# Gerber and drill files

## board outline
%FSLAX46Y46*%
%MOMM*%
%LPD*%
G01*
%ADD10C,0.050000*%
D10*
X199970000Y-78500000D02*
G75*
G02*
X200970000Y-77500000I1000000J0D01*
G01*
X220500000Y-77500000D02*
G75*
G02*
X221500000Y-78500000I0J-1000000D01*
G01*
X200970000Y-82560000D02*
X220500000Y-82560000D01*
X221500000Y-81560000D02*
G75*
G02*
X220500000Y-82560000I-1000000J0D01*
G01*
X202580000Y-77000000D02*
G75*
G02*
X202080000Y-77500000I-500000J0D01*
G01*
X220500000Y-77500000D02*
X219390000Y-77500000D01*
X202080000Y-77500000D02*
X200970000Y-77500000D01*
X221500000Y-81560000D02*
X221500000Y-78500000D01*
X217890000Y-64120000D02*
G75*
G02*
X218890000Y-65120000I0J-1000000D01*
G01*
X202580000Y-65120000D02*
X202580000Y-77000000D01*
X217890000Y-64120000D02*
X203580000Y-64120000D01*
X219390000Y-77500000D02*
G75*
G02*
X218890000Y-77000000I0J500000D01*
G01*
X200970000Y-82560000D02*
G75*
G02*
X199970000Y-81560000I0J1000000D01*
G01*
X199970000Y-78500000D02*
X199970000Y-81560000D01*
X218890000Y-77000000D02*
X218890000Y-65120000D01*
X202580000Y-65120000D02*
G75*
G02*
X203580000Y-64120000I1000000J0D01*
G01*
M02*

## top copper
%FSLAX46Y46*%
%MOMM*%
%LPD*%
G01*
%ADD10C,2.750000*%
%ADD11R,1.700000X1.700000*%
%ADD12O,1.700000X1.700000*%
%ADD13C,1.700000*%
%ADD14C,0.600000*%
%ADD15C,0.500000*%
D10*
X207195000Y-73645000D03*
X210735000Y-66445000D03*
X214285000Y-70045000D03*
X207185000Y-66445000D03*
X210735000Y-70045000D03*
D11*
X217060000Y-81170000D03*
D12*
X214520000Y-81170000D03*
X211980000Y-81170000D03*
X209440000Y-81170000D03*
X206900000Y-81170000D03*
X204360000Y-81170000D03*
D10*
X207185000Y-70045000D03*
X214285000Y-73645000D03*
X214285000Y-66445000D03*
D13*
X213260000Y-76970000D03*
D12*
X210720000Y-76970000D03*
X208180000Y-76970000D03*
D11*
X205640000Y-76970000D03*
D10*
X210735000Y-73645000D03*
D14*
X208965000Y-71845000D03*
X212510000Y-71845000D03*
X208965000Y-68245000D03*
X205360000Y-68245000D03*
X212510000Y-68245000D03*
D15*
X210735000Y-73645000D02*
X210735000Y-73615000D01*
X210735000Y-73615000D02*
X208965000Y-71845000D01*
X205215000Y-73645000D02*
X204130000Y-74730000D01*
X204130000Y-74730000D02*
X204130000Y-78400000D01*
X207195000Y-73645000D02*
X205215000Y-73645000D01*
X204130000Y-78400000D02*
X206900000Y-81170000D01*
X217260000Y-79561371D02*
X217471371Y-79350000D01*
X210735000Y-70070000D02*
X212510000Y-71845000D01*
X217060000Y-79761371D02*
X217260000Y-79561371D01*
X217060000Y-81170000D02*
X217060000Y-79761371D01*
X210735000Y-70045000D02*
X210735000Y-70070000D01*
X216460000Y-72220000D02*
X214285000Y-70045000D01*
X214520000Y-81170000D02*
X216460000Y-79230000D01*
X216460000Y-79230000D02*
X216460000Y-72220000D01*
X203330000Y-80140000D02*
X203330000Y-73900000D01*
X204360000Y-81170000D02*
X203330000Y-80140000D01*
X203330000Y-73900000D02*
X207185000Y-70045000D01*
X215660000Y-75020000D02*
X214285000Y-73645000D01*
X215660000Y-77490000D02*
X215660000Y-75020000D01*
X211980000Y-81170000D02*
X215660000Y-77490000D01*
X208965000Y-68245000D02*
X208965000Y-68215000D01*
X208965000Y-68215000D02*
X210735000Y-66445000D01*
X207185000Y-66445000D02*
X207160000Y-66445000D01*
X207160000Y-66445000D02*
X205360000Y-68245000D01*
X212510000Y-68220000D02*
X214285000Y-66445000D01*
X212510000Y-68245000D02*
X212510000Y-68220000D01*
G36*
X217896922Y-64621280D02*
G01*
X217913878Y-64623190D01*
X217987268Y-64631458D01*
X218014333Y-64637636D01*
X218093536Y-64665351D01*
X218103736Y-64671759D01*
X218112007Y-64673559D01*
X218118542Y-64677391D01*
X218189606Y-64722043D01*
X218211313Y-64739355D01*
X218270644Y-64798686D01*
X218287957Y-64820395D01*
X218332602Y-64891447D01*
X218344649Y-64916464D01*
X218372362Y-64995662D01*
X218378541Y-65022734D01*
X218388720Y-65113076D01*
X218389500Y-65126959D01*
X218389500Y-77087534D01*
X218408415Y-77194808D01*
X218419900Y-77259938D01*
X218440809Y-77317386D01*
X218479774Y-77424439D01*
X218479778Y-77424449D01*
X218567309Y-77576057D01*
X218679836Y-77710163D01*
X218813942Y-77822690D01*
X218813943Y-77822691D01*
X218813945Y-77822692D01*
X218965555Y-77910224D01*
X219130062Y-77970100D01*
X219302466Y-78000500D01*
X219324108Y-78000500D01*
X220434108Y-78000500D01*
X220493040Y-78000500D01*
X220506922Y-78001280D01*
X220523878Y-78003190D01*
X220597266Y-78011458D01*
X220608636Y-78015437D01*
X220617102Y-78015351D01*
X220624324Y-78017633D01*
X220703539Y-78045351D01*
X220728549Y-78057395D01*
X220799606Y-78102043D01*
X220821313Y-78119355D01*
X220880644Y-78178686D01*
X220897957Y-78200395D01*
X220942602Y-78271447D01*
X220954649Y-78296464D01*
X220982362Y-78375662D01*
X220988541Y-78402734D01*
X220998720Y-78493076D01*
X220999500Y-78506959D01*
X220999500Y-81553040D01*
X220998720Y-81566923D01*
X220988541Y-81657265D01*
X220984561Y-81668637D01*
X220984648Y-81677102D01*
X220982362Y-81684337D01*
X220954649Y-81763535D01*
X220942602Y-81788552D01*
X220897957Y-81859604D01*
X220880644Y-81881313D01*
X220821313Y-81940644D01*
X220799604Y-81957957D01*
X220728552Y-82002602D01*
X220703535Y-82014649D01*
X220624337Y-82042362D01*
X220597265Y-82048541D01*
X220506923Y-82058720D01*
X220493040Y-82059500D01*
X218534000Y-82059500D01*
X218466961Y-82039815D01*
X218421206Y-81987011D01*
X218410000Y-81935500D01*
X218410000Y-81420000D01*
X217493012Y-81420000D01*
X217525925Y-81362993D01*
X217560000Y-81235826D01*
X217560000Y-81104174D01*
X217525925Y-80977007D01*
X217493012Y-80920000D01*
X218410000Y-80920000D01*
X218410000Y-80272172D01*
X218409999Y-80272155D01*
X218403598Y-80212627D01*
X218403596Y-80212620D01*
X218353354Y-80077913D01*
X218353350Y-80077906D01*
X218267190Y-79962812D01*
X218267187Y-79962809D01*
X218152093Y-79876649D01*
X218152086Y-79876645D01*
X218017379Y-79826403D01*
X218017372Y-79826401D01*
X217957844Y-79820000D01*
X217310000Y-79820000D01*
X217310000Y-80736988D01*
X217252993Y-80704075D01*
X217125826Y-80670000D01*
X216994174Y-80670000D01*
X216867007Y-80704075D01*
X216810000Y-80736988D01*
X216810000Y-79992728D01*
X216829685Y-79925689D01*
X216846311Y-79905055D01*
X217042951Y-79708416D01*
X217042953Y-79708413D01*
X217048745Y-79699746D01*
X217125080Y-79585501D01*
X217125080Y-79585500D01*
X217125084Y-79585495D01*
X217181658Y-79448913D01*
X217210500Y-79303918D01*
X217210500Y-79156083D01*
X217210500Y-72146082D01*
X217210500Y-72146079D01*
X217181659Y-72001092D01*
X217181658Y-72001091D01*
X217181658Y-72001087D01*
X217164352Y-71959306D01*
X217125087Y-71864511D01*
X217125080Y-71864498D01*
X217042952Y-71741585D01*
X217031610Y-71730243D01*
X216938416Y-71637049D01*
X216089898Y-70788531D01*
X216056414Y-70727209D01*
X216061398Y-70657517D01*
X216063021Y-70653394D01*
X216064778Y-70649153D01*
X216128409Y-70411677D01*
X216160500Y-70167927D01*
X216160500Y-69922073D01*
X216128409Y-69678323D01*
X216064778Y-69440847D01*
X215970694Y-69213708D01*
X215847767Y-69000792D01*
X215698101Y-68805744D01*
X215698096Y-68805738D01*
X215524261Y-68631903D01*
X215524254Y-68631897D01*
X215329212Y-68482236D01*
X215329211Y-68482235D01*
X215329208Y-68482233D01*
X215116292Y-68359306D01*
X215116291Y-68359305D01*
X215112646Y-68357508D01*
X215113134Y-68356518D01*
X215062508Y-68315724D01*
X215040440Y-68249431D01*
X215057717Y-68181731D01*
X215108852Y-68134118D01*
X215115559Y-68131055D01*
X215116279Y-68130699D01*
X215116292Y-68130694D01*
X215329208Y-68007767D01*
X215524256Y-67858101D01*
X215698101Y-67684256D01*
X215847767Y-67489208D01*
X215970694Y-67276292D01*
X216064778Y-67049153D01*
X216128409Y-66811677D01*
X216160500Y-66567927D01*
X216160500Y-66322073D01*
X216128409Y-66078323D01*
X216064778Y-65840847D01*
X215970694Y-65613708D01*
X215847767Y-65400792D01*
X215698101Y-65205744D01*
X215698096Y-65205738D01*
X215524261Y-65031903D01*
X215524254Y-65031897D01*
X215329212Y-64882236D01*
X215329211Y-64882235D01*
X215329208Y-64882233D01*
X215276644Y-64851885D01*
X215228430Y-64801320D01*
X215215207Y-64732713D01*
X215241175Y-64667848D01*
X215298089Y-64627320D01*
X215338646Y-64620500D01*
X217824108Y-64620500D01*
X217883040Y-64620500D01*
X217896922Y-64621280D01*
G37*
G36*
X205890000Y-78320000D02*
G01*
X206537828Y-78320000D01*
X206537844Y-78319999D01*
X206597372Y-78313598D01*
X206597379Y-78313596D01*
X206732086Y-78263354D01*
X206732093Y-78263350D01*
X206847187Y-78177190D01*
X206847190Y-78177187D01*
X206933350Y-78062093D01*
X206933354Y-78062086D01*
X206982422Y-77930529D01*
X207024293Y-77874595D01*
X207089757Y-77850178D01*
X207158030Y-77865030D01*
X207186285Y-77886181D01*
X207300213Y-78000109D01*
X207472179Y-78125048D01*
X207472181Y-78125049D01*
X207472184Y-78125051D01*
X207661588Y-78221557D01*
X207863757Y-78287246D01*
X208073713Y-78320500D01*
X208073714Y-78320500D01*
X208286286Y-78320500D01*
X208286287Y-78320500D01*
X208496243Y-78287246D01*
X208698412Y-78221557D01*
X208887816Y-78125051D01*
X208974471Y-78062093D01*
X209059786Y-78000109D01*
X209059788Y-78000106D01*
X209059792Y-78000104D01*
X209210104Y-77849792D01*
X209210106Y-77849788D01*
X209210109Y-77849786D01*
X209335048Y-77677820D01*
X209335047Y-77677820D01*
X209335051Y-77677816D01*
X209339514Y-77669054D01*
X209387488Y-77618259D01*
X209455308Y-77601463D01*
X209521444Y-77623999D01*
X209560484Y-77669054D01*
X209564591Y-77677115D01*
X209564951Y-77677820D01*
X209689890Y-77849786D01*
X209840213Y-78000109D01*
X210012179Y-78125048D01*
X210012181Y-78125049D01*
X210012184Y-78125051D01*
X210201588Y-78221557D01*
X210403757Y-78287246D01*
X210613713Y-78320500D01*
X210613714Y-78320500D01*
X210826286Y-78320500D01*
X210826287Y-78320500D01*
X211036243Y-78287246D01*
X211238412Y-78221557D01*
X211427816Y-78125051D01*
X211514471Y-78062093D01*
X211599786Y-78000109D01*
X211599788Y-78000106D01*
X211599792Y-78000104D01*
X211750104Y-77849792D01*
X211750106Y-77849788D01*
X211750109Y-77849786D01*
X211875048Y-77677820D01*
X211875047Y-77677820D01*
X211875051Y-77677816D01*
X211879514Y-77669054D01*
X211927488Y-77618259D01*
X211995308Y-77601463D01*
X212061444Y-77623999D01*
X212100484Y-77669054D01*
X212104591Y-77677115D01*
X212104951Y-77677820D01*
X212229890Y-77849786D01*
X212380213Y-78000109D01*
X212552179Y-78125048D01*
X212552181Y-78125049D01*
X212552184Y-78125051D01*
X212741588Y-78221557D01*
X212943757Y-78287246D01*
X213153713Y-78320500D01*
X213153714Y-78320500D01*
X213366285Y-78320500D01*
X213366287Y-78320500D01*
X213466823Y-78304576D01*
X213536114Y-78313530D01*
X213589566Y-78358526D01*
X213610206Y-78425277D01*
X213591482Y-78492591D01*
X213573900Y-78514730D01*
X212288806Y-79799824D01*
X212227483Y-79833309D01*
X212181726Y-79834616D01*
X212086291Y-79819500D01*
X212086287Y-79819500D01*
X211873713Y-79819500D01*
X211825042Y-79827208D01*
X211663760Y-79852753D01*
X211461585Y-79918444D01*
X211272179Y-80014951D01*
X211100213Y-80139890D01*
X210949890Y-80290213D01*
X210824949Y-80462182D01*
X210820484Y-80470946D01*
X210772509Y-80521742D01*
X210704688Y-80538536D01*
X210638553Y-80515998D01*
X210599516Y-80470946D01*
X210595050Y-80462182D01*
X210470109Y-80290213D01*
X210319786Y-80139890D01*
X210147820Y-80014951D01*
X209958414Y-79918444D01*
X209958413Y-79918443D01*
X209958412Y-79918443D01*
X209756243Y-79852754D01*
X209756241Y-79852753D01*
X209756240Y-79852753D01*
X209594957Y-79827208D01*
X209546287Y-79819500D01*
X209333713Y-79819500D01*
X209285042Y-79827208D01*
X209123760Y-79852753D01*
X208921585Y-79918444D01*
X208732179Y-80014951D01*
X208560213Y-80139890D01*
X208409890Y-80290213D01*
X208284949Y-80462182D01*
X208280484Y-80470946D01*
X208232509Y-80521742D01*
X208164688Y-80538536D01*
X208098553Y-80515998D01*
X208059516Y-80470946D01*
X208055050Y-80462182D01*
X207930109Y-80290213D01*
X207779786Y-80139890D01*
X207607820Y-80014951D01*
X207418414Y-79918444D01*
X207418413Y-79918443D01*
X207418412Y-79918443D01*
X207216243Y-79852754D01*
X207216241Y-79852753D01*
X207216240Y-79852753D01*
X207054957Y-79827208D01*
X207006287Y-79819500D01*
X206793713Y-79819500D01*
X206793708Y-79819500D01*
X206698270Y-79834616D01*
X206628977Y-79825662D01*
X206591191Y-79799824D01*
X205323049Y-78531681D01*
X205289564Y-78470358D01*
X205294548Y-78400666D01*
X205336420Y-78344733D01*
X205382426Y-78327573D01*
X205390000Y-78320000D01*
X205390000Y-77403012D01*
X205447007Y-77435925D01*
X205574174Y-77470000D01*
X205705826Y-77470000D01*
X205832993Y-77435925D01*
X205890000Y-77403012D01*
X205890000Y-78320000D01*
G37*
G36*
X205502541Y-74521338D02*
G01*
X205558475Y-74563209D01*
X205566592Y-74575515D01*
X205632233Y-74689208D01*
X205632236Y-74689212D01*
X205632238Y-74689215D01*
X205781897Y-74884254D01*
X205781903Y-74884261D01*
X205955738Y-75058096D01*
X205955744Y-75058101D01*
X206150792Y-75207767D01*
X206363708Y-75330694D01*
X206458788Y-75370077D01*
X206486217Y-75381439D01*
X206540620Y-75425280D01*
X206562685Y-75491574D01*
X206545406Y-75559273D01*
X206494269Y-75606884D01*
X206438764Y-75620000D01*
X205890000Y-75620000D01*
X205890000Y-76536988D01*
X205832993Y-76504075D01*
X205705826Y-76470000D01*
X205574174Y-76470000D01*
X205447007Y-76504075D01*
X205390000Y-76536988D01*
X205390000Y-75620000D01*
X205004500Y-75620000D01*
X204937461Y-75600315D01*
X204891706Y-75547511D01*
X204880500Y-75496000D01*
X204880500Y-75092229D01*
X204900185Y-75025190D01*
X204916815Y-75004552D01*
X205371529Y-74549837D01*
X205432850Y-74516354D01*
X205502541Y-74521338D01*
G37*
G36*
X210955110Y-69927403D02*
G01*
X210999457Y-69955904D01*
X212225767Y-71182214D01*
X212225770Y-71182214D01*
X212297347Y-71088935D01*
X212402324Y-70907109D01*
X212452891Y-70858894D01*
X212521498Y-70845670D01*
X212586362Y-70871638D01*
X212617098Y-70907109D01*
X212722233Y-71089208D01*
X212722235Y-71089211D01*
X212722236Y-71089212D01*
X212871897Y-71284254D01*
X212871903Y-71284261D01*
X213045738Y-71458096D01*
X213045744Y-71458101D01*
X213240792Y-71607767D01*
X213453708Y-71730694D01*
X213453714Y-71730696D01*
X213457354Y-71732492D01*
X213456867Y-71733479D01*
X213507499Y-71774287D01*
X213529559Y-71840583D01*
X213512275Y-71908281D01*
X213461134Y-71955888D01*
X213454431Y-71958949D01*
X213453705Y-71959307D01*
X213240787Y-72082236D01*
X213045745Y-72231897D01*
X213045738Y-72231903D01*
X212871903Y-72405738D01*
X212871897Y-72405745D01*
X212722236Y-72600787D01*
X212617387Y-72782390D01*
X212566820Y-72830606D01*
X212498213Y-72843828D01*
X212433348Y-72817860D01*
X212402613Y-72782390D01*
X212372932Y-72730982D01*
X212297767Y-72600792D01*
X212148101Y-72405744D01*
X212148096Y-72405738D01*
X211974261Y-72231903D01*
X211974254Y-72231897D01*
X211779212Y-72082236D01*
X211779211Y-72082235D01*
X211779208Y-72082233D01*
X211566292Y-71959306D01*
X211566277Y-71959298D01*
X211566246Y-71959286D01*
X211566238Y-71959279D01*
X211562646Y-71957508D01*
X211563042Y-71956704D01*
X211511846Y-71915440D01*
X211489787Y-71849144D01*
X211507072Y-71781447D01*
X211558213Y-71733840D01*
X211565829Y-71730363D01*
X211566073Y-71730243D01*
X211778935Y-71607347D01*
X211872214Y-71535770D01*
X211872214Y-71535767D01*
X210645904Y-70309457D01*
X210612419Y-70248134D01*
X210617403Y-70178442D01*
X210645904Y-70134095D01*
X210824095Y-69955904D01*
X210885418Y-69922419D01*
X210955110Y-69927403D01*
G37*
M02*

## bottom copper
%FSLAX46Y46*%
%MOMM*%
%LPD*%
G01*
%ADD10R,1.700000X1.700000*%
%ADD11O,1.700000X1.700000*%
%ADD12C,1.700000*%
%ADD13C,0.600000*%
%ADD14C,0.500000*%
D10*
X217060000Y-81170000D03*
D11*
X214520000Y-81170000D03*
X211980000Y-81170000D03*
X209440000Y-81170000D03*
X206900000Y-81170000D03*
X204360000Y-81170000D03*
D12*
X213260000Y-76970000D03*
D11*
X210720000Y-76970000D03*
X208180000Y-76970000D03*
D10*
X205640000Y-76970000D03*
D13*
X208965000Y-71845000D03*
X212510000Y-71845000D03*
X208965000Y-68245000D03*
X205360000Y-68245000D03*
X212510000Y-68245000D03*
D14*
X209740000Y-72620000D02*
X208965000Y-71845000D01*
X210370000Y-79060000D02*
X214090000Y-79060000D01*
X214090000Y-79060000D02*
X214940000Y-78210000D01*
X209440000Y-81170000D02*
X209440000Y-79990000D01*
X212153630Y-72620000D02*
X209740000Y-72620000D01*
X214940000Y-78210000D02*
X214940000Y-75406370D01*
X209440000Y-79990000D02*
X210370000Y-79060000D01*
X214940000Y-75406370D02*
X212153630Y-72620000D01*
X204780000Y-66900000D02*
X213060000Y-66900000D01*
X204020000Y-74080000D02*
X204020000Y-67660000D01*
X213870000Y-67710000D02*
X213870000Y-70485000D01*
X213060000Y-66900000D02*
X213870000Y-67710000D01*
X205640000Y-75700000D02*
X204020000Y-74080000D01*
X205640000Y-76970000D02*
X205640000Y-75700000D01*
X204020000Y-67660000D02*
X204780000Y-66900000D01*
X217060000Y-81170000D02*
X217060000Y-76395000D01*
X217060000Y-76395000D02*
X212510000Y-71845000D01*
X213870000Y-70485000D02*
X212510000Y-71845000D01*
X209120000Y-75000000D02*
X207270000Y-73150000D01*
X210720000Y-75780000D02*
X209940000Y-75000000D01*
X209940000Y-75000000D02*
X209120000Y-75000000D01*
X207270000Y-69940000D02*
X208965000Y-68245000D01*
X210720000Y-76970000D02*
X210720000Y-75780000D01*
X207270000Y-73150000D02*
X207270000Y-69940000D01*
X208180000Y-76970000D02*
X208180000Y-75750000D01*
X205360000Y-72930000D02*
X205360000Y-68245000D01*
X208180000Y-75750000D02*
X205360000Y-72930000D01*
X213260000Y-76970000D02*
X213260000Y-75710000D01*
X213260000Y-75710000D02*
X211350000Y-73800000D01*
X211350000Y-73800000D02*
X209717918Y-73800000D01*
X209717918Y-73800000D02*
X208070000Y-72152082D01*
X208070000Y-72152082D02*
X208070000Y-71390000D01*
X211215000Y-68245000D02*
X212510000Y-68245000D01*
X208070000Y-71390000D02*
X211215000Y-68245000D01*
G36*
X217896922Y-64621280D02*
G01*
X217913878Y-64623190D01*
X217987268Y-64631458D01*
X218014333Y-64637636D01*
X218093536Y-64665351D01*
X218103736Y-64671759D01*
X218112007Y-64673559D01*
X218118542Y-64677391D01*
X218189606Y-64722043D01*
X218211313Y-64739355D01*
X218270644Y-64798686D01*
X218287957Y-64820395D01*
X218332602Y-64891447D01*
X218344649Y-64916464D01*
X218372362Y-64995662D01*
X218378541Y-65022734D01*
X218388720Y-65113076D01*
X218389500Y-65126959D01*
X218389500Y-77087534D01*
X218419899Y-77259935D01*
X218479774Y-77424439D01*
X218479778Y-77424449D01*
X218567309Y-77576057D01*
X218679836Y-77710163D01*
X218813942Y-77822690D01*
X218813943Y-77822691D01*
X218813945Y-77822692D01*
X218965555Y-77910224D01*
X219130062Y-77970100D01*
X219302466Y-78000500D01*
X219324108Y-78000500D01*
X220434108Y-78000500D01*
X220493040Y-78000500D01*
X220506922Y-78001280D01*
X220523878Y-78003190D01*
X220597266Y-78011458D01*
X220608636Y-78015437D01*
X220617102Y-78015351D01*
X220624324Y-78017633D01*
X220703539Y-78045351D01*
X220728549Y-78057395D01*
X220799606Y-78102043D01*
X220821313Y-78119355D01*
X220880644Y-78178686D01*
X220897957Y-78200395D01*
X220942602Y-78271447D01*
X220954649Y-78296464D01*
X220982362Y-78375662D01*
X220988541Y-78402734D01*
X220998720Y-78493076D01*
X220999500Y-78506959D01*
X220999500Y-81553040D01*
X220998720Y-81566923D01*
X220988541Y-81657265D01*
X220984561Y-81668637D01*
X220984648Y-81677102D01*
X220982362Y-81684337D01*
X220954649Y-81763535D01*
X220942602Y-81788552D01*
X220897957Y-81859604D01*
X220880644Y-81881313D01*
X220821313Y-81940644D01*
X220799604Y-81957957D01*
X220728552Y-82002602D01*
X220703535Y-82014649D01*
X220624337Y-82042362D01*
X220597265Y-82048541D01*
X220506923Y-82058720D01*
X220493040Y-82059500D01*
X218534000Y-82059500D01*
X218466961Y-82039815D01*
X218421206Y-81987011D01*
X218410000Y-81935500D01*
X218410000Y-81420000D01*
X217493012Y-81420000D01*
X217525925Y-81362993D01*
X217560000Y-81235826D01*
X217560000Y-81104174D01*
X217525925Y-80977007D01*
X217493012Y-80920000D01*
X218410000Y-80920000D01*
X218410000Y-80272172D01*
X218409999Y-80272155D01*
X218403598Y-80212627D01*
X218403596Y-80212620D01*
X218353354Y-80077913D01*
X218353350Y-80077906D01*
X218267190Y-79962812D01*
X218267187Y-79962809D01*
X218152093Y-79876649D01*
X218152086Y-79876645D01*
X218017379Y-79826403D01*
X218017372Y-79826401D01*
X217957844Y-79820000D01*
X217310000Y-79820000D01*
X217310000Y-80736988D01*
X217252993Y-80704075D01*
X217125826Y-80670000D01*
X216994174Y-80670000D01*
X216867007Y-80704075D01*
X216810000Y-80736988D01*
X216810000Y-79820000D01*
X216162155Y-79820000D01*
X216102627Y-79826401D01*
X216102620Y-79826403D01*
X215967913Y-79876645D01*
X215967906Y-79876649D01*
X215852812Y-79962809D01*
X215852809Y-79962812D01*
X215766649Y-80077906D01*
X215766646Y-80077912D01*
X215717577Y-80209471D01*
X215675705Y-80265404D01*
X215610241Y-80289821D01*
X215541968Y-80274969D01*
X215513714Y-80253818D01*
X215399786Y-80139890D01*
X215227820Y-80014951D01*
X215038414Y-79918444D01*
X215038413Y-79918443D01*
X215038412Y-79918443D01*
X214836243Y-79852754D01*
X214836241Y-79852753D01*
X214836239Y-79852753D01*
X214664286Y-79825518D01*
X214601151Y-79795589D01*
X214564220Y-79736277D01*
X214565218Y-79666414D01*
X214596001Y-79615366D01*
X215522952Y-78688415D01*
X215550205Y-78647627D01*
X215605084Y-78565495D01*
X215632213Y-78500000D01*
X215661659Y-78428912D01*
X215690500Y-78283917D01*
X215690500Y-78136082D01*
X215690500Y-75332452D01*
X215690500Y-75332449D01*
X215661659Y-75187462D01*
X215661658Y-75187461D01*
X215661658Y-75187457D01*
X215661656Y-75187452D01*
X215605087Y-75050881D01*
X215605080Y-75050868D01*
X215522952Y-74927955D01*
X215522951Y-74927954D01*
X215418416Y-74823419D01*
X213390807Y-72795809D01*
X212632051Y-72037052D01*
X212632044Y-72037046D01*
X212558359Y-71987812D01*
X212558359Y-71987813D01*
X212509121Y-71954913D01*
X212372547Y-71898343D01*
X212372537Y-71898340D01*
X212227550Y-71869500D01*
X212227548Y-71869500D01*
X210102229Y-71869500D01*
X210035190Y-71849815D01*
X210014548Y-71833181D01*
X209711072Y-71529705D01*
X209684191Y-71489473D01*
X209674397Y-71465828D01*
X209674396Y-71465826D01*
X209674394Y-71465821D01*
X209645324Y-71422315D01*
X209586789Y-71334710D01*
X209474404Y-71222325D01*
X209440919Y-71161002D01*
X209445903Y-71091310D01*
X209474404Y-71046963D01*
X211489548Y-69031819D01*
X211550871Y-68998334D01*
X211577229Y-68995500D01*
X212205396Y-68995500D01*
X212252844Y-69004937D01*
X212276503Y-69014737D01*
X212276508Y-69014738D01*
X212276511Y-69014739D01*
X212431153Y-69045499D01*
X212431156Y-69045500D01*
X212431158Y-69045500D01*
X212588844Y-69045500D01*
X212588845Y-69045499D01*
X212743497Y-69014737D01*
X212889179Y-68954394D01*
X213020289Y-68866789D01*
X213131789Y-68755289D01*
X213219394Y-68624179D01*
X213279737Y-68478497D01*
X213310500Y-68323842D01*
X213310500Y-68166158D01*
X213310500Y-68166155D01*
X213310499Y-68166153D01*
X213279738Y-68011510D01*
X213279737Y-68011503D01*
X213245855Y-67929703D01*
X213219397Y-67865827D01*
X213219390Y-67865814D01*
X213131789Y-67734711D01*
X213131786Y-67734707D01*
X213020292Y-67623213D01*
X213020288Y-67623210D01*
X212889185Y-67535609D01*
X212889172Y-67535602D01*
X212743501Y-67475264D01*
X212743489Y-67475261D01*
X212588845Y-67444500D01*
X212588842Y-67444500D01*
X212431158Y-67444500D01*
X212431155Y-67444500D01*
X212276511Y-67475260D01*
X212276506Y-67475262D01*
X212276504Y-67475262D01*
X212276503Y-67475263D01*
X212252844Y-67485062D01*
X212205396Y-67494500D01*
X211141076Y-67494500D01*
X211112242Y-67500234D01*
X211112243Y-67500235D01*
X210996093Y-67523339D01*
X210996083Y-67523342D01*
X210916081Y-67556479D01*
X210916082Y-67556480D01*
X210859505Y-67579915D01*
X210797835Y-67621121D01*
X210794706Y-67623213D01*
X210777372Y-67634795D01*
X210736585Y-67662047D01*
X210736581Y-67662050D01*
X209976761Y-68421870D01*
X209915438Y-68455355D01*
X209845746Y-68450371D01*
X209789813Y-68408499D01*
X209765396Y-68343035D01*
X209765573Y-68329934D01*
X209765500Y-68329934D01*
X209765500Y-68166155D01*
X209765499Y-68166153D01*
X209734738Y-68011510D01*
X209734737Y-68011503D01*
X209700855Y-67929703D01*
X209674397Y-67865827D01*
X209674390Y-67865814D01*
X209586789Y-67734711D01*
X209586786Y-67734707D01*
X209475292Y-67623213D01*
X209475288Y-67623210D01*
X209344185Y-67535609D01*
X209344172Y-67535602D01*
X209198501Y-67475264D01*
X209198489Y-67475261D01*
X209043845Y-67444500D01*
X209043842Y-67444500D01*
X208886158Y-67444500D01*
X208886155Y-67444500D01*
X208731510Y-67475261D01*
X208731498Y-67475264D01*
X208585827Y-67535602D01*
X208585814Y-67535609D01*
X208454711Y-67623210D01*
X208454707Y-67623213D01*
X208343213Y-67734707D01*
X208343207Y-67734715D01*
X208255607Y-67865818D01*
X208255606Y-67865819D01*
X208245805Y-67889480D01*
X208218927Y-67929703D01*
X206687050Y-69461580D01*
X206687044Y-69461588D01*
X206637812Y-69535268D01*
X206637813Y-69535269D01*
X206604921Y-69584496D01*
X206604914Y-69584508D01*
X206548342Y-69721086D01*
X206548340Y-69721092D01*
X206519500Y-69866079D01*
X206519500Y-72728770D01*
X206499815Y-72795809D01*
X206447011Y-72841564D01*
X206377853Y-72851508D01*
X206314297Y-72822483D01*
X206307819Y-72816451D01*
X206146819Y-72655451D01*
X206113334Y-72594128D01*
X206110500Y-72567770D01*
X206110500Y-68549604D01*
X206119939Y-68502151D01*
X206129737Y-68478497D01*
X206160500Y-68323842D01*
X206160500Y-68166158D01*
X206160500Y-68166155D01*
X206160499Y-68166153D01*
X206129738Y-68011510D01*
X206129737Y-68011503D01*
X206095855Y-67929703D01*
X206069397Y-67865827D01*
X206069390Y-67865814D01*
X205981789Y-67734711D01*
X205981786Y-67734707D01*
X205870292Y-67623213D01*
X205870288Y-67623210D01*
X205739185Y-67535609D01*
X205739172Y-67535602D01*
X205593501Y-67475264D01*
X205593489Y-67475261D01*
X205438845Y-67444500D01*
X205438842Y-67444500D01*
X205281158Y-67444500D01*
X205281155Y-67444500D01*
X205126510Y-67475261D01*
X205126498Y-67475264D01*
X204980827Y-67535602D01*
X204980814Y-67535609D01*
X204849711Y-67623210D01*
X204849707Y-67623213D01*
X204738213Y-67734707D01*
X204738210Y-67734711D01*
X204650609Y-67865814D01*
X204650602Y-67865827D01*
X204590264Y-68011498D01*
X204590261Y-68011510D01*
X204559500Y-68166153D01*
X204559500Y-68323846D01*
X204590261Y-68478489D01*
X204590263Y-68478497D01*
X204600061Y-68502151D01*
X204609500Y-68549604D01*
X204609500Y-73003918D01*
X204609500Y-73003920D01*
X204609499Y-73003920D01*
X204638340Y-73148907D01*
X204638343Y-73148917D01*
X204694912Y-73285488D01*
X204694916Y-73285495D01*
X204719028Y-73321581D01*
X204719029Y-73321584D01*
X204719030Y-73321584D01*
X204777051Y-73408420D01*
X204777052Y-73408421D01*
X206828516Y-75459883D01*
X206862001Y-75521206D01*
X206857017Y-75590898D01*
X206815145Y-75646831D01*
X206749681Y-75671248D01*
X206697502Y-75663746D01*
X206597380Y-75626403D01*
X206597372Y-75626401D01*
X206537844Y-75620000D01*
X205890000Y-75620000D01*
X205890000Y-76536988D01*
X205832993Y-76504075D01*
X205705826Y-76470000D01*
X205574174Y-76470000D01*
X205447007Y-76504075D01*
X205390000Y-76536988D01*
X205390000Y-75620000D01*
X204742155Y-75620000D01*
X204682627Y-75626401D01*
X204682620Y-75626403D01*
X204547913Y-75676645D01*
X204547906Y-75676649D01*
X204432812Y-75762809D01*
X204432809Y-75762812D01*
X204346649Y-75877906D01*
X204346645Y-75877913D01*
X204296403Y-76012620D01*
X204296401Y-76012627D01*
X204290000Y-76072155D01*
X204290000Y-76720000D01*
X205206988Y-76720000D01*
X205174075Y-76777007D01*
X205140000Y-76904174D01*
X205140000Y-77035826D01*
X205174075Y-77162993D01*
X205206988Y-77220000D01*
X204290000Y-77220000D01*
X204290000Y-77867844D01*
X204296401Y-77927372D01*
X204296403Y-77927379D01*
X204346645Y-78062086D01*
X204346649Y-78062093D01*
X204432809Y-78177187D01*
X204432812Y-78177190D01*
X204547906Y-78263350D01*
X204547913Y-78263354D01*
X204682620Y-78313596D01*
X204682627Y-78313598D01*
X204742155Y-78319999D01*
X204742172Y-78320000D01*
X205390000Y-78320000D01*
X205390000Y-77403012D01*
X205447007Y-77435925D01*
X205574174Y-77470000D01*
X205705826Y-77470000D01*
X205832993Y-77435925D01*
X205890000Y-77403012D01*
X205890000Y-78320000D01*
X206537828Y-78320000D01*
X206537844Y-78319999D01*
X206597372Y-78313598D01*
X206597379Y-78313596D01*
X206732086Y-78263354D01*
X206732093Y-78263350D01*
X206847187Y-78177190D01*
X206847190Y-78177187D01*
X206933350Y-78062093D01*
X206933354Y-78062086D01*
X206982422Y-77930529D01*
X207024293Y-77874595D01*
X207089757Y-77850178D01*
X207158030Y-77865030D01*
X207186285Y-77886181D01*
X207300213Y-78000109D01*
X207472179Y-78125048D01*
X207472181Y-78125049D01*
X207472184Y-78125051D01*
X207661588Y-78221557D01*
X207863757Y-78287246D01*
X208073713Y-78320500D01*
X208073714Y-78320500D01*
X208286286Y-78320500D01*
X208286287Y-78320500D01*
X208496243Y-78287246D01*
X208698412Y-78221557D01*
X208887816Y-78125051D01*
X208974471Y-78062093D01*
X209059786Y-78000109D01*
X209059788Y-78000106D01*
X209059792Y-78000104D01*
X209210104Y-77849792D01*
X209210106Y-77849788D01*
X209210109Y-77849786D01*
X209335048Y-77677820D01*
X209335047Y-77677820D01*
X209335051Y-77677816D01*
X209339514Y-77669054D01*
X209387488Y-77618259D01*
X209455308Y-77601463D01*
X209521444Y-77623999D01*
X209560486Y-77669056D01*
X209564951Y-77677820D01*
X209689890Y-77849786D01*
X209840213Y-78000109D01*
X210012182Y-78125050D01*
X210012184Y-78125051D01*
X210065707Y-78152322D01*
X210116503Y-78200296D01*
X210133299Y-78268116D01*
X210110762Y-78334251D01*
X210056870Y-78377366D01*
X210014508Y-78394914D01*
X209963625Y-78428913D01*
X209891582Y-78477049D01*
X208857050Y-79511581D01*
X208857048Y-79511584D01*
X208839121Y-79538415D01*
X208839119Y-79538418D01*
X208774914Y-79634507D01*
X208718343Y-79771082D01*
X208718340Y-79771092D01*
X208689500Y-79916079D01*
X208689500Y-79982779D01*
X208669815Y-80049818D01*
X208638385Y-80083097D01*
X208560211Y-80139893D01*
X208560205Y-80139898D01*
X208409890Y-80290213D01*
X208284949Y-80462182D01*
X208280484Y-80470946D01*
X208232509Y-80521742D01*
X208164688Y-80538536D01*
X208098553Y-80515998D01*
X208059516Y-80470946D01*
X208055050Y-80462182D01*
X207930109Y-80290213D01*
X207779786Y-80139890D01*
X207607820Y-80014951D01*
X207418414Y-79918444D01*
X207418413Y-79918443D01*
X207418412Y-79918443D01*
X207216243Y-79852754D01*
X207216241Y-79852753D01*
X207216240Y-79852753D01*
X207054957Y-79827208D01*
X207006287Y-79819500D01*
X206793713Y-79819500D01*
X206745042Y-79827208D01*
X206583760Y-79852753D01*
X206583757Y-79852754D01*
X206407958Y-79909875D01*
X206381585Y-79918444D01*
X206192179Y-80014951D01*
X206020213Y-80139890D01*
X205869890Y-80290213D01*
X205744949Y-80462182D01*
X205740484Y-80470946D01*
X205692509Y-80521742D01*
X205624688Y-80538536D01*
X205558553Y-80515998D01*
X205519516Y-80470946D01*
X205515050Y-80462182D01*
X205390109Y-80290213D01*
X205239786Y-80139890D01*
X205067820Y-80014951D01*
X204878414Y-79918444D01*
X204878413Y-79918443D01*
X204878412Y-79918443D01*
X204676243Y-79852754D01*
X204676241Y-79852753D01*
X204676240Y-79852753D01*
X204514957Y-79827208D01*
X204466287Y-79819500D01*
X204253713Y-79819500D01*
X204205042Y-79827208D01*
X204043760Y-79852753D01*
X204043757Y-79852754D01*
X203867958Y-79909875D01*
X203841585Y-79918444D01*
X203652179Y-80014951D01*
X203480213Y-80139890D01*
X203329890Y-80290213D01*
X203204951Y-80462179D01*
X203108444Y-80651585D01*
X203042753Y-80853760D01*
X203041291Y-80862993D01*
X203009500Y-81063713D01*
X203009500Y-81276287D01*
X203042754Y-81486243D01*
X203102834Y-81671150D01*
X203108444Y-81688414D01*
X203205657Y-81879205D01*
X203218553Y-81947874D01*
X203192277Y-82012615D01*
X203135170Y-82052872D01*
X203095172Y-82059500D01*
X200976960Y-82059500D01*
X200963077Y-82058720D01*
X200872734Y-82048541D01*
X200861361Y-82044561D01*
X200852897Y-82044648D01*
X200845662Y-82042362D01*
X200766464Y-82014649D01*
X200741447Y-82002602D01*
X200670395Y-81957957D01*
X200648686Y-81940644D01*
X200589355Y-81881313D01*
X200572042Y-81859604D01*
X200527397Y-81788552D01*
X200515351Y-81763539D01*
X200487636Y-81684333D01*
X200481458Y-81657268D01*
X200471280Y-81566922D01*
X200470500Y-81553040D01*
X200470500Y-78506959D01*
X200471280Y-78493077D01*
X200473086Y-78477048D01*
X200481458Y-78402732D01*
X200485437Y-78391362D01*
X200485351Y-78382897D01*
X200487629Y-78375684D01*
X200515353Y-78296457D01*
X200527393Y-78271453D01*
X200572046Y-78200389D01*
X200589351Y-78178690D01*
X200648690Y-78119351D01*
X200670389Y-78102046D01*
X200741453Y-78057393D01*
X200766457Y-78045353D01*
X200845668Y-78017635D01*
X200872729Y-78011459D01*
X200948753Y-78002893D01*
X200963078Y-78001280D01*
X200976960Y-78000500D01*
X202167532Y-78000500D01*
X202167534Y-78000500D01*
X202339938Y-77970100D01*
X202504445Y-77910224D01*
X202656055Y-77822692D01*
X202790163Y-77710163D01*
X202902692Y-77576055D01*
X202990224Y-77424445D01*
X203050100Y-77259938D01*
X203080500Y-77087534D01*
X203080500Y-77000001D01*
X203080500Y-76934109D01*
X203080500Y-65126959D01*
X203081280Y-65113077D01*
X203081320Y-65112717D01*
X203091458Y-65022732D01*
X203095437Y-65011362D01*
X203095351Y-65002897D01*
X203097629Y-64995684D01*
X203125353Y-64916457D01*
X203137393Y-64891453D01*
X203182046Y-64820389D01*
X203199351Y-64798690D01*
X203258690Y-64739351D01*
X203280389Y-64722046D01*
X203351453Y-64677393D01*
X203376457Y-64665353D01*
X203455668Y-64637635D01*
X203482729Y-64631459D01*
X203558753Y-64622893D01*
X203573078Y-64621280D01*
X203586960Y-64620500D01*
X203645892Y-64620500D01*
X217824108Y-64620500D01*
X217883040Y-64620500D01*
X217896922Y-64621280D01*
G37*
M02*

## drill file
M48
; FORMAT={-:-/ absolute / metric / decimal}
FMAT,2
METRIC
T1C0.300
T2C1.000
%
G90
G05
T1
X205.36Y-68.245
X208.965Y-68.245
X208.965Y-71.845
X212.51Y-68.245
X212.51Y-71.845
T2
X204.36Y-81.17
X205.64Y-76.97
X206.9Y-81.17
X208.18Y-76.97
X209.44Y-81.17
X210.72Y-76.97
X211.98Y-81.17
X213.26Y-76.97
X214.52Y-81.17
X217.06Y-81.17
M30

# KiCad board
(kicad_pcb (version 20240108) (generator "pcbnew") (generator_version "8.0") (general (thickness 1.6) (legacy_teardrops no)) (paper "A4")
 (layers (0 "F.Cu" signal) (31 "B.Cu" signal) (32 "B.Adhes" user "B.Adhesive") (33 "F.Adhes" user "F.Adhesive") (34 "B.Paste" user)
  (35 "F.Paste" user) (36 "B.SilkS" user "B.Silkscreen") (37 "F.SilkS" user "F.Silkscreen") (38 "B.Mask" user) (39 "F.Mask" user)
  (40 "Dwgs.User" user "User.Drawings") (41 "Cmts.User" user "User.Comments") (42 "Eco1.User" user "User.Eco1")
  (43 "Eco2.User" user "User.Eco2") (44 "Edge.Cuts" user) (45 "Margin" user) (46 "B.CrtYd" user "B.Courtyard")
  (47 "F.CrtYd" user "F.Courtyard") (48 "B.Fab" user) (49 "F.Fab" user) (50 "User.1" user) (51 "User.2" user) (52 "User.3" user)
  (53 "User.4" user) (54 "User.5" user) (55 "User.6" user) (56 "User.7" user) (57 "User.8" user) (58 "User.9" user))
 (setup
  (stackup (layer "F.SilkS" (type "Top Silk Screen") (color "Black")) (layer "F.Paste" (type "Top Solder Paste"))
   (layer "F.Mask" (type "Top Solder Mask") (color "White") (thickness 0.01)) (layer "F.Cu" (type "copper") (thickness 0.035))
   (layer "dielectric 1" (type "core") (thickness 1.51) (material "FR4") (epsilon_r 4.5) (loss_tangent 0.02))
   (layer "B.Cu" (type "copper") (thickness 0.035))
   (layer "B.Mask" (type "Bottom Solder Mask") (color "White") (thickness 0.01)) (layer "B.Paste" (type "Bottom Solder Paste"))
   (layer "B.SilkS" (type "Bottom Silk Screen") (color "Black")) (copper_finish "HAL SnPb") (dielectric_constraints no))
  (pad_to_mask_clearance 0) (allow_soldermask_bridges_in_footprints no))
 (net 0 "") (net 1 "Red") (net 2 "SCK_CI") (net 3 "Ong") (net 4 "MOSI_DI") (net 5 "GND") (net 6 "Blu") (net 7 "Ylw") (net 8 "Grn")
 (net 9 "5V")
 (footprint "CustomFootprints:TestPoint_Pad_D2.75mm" (layer "F.Cu") (at 207.195 73.645)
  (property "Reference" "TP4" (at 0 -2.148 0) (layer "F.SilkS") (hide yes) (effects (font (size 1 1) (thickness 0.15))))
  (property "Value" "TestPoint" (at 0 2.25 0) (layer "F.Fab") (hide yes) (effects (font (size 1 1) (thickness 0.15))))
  (pad "1" smd circle (at 0 0) (size 2.75 2.75) (layers "F.Cu" "F.Mask") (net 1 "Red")))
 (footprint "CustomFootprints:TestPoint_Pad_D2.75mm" (layer "F.Cu") (at 210.735 66.445)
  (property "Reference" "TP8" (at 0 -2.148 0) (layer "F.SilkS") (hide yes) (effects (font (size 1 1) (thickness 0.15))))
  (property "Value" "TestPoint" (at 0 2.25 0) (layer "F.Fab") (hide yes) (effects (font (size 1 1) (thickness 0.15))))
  (pad "1" smd circle (at 0 0) (size 2.75 2.75) (layers "F.Cu" "F.Mask") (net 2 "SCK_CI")))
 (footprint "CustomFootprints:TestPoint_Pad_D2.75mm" (layer "F.Cu") (at 214.285 70.045)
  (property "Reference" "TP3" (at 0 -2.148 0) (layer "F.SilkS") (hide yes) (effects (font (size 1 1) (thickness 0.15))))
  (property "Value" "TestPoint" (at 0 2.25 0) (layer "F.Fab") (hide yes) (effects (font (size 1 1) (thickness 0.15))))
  (pad "1" smd circle (at 0 0) (size 2.75 2.75) (layers "F.Cu" "F.Mask") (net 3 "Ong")))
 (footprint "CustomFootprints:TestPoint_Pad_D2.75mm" (layer "F.Cu") (at 207.185 66.445)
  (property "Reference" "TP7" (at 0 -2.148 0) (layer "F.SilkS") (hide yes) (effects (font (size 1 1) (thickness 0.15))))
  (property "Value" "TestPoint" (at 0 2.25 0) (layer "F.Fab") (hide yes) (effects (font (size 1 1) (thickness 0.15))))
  (pad "1" smd circle (at 0 0) (size 2.75 2.75) (layers "F.Cu" "F.Mask") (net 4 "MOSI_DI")))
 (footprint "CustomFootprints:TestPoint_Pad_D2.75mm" (layer "F.Cu") (at 210.735 70.045)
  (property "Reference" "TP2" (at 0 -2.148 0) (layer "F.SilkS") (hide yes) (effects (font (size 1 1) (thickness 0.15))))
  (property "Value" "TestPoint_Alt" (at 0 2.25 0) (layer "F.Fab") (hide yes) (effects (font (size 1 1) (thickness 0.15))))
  (pad "1" smd circle (at 0 0) (size 2.75 2.75) (layers "F.Cu" "F.Mask") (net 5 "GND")))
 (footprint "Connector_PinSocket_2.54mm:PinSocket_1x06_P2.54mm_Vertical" (layer "F.Cu") (at 217.06 81.17 -90)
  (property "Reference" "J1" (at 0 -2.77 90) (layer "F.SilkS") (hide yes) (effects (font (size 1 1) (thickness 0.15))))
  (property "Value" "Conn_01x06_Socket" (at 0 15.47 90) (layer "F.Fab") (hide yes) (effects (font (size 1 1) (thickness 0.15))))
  (pad "1" thru_hole rect (at 0 0 270) (size 1.7 1.7) (drill 1) (layers "*.Cu" "*.Mask") (remove_unused_layers no) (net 5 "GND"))
  (pad "2" thru_hole oval (at 0 2.54 270) (size 1.7 1.7) (drill 1) (layers "*.Cu" "*.Mask") (remove_unused_layers no) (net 3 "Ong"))
  (pad "3" thru_hole oval (at 0 5.08 270) (size 1.7 1.7) (drill 1) (layers "*.Cu" "*.Mask") (remove_unused_layers no) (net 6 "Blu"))
  (pad "4" thru_hole oval (at 0 7.62 270) (size 1.7 1.7) (drill 1) (layers "*.Cu" "*.Mask") (remove_unused_layers no) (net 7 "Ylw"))
  (pad "5" thru_hole oval (at 0 10.16 270) (size 1.7 1.7) (drill 1) (layers "*.Cu" "*.Mask") (remove_unused_layers no) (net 1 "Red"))
  (pad "6" thru_hole oval (at 0 12.7 270) (size 1.7 1.7) (drill 1) (layers "*.Cu" "*.Mask") (remove_unused_layers no) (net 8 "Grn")))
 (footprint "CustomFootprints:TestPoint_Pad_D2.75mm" (layer "F.Cu") (at 207.185 70.045)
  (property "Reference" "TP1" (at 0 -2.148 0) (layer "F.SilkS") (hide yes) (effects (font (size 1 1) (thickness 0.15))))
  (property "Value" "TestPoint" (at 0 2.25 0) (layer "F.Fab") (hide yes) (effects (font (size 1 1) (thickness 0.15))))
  (pad "1" smd circle (at 0 0) (size 2.75 2.75) (layers "F.Cu" "F.Mask") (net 8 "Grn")))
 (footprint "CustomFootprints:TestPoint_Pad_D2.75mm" (layer "F.Cu") (at 214.285 73.645)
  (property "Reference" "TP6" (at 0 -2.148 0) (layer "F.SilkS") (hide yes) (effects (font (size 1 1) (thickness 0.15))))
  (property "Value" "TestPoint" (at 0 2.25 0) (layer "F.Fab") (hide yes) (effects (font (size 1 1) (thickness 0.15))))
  (pad "1" smd circle (at 0 0) (size 2.75 2.75) (layers "F.Cu" "F.Mask") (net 6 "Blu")))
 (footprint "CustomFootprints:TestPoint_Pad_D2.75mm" (layer "F.Cu") (at 214.285 66.445)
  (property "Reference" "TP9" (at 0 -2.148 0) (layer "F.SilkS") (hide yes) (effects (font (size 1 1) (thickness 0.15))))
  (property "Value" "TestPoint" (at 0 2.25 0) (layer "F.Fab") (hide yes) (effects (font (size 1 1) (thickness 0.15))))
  (pad "1" smd circle (at 0 0) (size 2.75 2.75) (layers "F.Cu" "F.Mask") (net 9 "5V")))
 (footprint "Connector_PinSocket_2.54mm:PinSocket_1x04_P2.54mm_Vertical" (layer "F.Cu") (at 213.26 76.97 -90)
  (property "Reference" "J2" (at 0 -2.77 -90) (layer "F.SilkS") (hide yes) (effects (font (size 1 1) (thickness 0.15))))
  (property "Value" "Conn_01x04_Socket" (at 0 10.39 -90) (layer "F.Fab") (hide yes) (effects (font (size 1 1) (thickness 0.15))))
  (pad "1" thru_hole circle (at 0 0 270) (size 1.7 1.7) (drill 1) (layers "*.Cu" "*.Mask") (remove_unused_layers no) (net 9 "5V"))
  (pad "2" thru_hole oval (at 0 2.54 270) (size 1.7 1.7) (drill 1) (layers "*.Cu" "*.Mask") (remove_unused_layers no) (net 2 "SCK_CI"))
  (pad "3" thru_hole oval (at 0 5.08 270) (size 1.7 1.7) (drill 1) (layers "*.Cu" "*.Mask") (remove_unused_layers no) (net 4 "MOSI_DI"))
  (pad "4" thru_hole rect (at 0 7.62 270) (size 1.7 1.7) (drill 1) (layers "*.Cu" "*.Mask") (remove_unused_layers no) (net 5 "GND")))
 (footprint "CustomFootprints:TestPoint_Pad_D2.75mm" (layer "F.Cu") (at 210.735 73.645)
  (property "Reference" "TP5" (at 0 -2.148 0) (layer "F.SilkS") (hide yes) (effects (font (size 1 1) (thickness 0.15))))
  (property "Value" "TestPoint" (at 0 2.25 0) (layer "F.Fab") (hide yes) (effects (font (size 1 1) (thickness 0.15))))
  (pad "1" smd circle (at 0 0) (size 2.75 2.75) (layers "F.Cu" "F.Mask") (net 7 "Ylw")))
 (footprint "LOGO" (layer "B.Cu") (at 210.671923 70.060189 180)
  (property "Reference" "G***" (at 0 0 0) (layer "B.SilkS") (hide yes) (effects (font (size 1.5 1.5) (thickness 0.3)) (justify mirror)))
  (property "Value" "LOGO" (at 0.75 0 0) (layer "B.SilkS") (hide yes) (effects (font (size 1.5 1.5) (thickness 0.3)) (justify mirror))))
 (gr_arc (start 199.97 78.5) (mid 200.262893 77.792893) (end 200.97 77.5) (stroke (width 0.05) (type default)) (layer "Edge.Cuts"))
 (gr_arc (start 220.5 77.5) (mid 221.207107 77.792893) (end 221.5 78.5) (stroke (width 0.05) (type default)) (layer "Edge.Cuts"))
 (gr_line (start 200.97 82.56) (end 220.5 82.56) (stroke (width 0.05) (type default)) (layer "Edge.Cuts"))
 (gr_arc (start 221.5 81.56) (mid 221.207107 82.267107) (end 220.5 82.56) (stroke (width 0.05) (type default)) (layer "Edge.Cuts"))
 (gr_arc (start 202.58 77) (mid 202.433553 77.353553) (end 202.08 77.5) (stroke (width 0.05) (type default)) (layer "Edge.Cuts"))
 (gr_line (start 220.5 77.5) (end 219.39 77.5) (stroke (width 0.05) (type default)) (layer "Edge.Cuts"))
 (gr_line (start 202.08 77.5) (end 200.97 77.5) (stroke (width 0.05) (type default)) (layer "Edge.Cuts"))
 (gr_line (start 221.5 81.56) (end 221.5 78.5) (stroke (width 0.05) (type default)) (layer "Edge.Cuts"))
 (gr_arc (start 217.89 64.12) (mid 218.597107 64.412893) (end 218.89 65.12) (stroke (width 0.05) (type default)) (layer "Edge.Cuts"))
 (gr_line (start 202.58 65.12) (end 202.58 77) (stroke (width 0.05) (type default)) (layer "Edge.Cuts"))
 (gr_line (start 217.89 64.12) (end 203.58 64.12) (stroke (width 0.05) (type default)) (layer "Edge.Cuts"))
 (gr_arc (start 219.39 77.5) (mid 219.036447 77.353553) (end 218.89 77) (stroke (width 0.05) (type default)) (layer "Edge.Cuts"))
 (gr_arc (start 200.97 82.56) (mid 200.262893 82.267107) (end 199.97 81.56) (stroke (width 0.05) (type default)) (layer "Edge.Cuts"))
 (gr_line (start 199.97 78.5) (end 199.97 81.56) (stroke (width 0.05) (type default)) (layer "Edge.Cuts"))
 (gr_line (start 218.89 77) (end 218.89 65.12) (stroke (width 0.05) (type default)) (layer "Edge.Cuts"))
 (gr_arc (start 202.58 65.12) (mid 202.872893 64.412893) (end 203.58 64.12) (stroke (width 0.05) (type default)) (layer "Edge.Cuts"))
 (segment (start 210.735 73.645) (end 210.735 73.615) (width 0.5) (layer "F.Cu") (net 7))
 (segment (start 210.735 73.615) (end 208.965 71.845) (width 0.5) (layer "F.Cu") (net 7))
 (via (at 208.965 71.845) (size 0.6) (drill 0.3) (layers "F.Cu" "B.Cu") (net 7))
 (segment (start 209.74 72.62) (end 208.965 71.845) (width 0.5) (layer "B.Cu") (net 7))
 (segment (start 210.37 79.06) (end 214.09 79.06) (width 0.5) (layer "B.Cu") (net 7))
 (segment (start 214.09 79.06) (end 214.94 78.21) (width 0.5) (layer "B.Cu") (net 7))
 (segment (start 209.44 81.17) (end 209.44 79.99) (width 0.5) (layer "B.Cu") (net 7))
 (segment (start 212.15363 72.62) (end 209.74 72.62) (width 0.5) (layer "B.Cu") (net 7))
 (segment (start 214.94 78.21) (end 214.94 75.40637) (width 0.5) (layer "B.Cu") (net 7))
 (segment (start 209.44 79.99) (end 210.37 79.06) (width 0.5) (layer "B.Cu") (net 7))
 (segment (start 214.94 75.40637) (end 212.15363 72.62) (width 0.5) (layer "B.Cu") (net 7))
 (segment (start 205.215 73.645) (end 204.13 74.73) (width 0.5) (layer "F.Cu") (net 1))
 (segment (start 204.13 74.73) (end 204.13 78.4) (width 0.5) (layer "F.Cu") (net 1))
 (segment (start 207.195 73.645) (end 205.215 73.645) (width 0.5) (layer "F.Cu") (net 1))
 (segment (start 204.13 78.4) (end 206.9 81.17) (width 0.5) (layer "F.Cu") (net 1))
 (segment (start 217.26 79.561371) (end 217.471371 79.35) (width 0.5) (layer "F.Cu") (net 5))
 (segment (start 210.735 70.07) (end 212.51 71.845) (width 0.5) (layer "F.Cu") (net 5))
 (segment (start 217.06 79.761371) (end 217.26 79.561371) (width 0.5) (layer "F.Cu") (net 5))
 (segment (start 217.06 81.17) (end 217.06 79.761371) (width 0.5) (layer "F.Cu") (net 5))
 (segment (start 210.735 70.045) (end 210.735 70.07) (width 0.5) (layer "F.Cu") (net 5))
 (via (at 212.51 71.845) (size 0.6) (drill 0.3) (layers "F.Cu" "B.Cu") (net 5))
 (segment (start 204.78 66.9) (end 213.06 66.9) (width 0.5) (layer "B.Cu") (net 5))
 (segment (start 204.02 74.08) (end 204.02 67.66) (width 0.5) (layer "B.Cu") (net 5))
 (segment (start 213.87 67.71) (end 213.87 70.485) (width 0.5) (layer "B.Cu") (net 5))
 (segment (start 213.06 66.9) (end 213.87 67.71) (width 0.5) (layer "B.Cu") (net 5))
 (segment (start 205.64 75.7) (end 204.02 74.08) (width 0.5) (layer "B.Cu") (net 5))
 (segment (start 205.64 76.97) (end 205.64 75.7) (width 0.5) (layer "B.Cu") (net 5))
 (segment (start 204.02 67.66) (end 204.78 66.9) (width 0.5) (layer "B.Cu") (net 5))
 (segment (start 217.06 81.17) (end 217.06 76.395) (width 0.5) (layer "B.Cu") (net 5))
 (segment (start 217.06 76.395) (end 212.51 71.845) (width 0.5) (layer "B.Cu") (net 5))
 (segment (start 213.87 70.485) (end 212.51 71.845) (width 0.5) (layer "B.Cu") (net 5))
 (segment (start 216.46 72.22) (end 214.285 70.045) (width 0.5) (layer "F.Cu") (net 3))
 (segment (start 214.52 81.17) (end 216.46 79.23) (width 0.5) (layer "F.Cu") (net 3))
 (segment (start 216.46 79.23) (end 216.46 72.22) (width 0.5) (layer "F.Cu") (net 3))
 (segment (start 203.33 80.14) (end 203.33 73.9) (width 0.5) (layer "F.Cu") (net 8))
 (segment (start 204.36 81.17) (end 203.33 80.14) (width 0.5) (layer "F.Cu") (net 8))
 (segment (start 203.33 73.9) (end 207.185 70.045) (width 0.5) (layer "F.Cu") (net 8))
 (segment (start 215.66 75.02) (end 214.285 73.645) (width 0.5) (layer "F.Cu") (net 6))
 (segment (start 215.66 77.49) (end 215.66 75.02) (width 0.5) (layer "F.Cu") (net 6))
 (segment (start 211.98 81.17) (end 215.66 77.49) (width 0.5) (layer "F.Cu") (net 6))
 (segment (start 208.965 68.245) (end 208.965 68.215) (width 0.5) (layer "F.Cu") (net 2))
 (segment (start 208.965 68.215) (end 210.735 66.445) (width 0.5) (layer "F.Cu") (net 2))
 (via (at 208.965 68.245) (size 0.6) (drill 0.3) (layers "F.Cu" "B.Cu") (locked yes) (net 2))
 (segment (start 209.12 75) (end 207.27 73.15) (width 0.5) (layer "B.Cu") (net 2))
 (segment (start 210.72 75.78) (end 209.94 75) (width 0.5) (layer "B.Cu") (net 2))
 (segment (start 209.94 75) (end 209.12 75) (width 0.5) (layer "B.Cu") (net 2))
 (segment (start 207.27 69.94) (end 208.965 68.245) (width 0.5) (layer "B.Cu") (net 2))
 (segment (start 210.72 76.97) (end 210.72 75.78) (width 0.5) (layer "B.Cu") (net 2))
 (segment (start 207.27 73.15) (end 207.27 69.94) (width 0.5) (layer "B.Cu") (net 2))
 (segment (start 207.185 66.445) (end 207.16 66.445) (width 0.5) (layer "F.Cu") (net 4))
 (segment (start 207.16 66.445) (end 205.36 68.245) (width 0.5) (layer "F.Cu") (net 4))
 (via (at 205.36 68.245) (size 0.6) (drill 0.3) (layers "F.Cu" "B.Cu") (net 4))
 (segment (start 208.18 76.97) (end 208.18 75.75) (width 0.5) (layer "B.Cu") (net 4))
 (segment (start 205.36 72.93) (end 205.36 68.245) (width 0.5) (layer "B.Cu") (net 4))
 (segment (start 208.18 75.75) (end 205.36 72.93) (width 0.5) (layer "B.Cu") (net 4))
 (segment (start 212.51 68.22) (end 214.285 66.445) (width 0.5) (layer "F.Cu") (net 9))
 (segment (start 212.51 68.245) (end 212.51 68.22) (width 0.5) (layer "F.Cu") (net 9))
 (via (at 212.51 68.245) (size 0.6) (drill 0.3) (layers "F.Cu" "B.Cu") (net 9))
 (segment (start 213.26 76.97) (end 213.26 75.71) (width 0.5) (layer "B.Cu") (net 9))
 (segment (start 213.26 75.71) (end 211.35 73.8) (width 0.5) (layer "B.Cu") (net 9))
 (segment (start 211.35 73.8) (end 209.717918 73.8) (width 0.5) (layer "B.Cu") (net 9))
 (segment (start 209.717918 73.8) (end 208.07 72.152082) (width 0.5) (layer "B.Cu") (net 9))
 (segment (start 208.07 72.152082) (end 208.07 71.39) (width 0.5) (layer "B.Cu") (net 9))
 (segment (start 211.215 68.245) (end 212.51 68.245) (width 0.5) (layer "B.Cu") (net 9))
 (segment (start 208.07 71.39) (end 211.215 68.245) (width 0.5) (layer "B.Cu") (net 9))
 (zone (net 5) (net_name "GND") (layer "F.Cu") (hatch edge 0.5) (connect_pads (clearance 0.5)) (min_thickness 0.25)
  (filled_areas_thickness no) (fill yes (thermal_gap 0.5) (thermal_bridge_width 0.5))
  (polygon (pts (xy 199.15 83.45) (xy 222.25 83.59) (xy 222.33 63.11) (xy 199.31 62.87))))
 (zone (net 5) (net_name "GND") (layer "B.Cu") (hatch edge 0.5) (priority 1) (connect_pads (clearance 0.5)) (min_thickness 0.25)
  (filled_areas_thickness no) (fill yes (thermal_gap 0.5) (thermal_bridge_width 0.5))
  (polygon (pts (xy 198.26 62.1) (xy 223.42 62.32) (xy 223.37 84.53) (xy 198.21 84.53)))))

